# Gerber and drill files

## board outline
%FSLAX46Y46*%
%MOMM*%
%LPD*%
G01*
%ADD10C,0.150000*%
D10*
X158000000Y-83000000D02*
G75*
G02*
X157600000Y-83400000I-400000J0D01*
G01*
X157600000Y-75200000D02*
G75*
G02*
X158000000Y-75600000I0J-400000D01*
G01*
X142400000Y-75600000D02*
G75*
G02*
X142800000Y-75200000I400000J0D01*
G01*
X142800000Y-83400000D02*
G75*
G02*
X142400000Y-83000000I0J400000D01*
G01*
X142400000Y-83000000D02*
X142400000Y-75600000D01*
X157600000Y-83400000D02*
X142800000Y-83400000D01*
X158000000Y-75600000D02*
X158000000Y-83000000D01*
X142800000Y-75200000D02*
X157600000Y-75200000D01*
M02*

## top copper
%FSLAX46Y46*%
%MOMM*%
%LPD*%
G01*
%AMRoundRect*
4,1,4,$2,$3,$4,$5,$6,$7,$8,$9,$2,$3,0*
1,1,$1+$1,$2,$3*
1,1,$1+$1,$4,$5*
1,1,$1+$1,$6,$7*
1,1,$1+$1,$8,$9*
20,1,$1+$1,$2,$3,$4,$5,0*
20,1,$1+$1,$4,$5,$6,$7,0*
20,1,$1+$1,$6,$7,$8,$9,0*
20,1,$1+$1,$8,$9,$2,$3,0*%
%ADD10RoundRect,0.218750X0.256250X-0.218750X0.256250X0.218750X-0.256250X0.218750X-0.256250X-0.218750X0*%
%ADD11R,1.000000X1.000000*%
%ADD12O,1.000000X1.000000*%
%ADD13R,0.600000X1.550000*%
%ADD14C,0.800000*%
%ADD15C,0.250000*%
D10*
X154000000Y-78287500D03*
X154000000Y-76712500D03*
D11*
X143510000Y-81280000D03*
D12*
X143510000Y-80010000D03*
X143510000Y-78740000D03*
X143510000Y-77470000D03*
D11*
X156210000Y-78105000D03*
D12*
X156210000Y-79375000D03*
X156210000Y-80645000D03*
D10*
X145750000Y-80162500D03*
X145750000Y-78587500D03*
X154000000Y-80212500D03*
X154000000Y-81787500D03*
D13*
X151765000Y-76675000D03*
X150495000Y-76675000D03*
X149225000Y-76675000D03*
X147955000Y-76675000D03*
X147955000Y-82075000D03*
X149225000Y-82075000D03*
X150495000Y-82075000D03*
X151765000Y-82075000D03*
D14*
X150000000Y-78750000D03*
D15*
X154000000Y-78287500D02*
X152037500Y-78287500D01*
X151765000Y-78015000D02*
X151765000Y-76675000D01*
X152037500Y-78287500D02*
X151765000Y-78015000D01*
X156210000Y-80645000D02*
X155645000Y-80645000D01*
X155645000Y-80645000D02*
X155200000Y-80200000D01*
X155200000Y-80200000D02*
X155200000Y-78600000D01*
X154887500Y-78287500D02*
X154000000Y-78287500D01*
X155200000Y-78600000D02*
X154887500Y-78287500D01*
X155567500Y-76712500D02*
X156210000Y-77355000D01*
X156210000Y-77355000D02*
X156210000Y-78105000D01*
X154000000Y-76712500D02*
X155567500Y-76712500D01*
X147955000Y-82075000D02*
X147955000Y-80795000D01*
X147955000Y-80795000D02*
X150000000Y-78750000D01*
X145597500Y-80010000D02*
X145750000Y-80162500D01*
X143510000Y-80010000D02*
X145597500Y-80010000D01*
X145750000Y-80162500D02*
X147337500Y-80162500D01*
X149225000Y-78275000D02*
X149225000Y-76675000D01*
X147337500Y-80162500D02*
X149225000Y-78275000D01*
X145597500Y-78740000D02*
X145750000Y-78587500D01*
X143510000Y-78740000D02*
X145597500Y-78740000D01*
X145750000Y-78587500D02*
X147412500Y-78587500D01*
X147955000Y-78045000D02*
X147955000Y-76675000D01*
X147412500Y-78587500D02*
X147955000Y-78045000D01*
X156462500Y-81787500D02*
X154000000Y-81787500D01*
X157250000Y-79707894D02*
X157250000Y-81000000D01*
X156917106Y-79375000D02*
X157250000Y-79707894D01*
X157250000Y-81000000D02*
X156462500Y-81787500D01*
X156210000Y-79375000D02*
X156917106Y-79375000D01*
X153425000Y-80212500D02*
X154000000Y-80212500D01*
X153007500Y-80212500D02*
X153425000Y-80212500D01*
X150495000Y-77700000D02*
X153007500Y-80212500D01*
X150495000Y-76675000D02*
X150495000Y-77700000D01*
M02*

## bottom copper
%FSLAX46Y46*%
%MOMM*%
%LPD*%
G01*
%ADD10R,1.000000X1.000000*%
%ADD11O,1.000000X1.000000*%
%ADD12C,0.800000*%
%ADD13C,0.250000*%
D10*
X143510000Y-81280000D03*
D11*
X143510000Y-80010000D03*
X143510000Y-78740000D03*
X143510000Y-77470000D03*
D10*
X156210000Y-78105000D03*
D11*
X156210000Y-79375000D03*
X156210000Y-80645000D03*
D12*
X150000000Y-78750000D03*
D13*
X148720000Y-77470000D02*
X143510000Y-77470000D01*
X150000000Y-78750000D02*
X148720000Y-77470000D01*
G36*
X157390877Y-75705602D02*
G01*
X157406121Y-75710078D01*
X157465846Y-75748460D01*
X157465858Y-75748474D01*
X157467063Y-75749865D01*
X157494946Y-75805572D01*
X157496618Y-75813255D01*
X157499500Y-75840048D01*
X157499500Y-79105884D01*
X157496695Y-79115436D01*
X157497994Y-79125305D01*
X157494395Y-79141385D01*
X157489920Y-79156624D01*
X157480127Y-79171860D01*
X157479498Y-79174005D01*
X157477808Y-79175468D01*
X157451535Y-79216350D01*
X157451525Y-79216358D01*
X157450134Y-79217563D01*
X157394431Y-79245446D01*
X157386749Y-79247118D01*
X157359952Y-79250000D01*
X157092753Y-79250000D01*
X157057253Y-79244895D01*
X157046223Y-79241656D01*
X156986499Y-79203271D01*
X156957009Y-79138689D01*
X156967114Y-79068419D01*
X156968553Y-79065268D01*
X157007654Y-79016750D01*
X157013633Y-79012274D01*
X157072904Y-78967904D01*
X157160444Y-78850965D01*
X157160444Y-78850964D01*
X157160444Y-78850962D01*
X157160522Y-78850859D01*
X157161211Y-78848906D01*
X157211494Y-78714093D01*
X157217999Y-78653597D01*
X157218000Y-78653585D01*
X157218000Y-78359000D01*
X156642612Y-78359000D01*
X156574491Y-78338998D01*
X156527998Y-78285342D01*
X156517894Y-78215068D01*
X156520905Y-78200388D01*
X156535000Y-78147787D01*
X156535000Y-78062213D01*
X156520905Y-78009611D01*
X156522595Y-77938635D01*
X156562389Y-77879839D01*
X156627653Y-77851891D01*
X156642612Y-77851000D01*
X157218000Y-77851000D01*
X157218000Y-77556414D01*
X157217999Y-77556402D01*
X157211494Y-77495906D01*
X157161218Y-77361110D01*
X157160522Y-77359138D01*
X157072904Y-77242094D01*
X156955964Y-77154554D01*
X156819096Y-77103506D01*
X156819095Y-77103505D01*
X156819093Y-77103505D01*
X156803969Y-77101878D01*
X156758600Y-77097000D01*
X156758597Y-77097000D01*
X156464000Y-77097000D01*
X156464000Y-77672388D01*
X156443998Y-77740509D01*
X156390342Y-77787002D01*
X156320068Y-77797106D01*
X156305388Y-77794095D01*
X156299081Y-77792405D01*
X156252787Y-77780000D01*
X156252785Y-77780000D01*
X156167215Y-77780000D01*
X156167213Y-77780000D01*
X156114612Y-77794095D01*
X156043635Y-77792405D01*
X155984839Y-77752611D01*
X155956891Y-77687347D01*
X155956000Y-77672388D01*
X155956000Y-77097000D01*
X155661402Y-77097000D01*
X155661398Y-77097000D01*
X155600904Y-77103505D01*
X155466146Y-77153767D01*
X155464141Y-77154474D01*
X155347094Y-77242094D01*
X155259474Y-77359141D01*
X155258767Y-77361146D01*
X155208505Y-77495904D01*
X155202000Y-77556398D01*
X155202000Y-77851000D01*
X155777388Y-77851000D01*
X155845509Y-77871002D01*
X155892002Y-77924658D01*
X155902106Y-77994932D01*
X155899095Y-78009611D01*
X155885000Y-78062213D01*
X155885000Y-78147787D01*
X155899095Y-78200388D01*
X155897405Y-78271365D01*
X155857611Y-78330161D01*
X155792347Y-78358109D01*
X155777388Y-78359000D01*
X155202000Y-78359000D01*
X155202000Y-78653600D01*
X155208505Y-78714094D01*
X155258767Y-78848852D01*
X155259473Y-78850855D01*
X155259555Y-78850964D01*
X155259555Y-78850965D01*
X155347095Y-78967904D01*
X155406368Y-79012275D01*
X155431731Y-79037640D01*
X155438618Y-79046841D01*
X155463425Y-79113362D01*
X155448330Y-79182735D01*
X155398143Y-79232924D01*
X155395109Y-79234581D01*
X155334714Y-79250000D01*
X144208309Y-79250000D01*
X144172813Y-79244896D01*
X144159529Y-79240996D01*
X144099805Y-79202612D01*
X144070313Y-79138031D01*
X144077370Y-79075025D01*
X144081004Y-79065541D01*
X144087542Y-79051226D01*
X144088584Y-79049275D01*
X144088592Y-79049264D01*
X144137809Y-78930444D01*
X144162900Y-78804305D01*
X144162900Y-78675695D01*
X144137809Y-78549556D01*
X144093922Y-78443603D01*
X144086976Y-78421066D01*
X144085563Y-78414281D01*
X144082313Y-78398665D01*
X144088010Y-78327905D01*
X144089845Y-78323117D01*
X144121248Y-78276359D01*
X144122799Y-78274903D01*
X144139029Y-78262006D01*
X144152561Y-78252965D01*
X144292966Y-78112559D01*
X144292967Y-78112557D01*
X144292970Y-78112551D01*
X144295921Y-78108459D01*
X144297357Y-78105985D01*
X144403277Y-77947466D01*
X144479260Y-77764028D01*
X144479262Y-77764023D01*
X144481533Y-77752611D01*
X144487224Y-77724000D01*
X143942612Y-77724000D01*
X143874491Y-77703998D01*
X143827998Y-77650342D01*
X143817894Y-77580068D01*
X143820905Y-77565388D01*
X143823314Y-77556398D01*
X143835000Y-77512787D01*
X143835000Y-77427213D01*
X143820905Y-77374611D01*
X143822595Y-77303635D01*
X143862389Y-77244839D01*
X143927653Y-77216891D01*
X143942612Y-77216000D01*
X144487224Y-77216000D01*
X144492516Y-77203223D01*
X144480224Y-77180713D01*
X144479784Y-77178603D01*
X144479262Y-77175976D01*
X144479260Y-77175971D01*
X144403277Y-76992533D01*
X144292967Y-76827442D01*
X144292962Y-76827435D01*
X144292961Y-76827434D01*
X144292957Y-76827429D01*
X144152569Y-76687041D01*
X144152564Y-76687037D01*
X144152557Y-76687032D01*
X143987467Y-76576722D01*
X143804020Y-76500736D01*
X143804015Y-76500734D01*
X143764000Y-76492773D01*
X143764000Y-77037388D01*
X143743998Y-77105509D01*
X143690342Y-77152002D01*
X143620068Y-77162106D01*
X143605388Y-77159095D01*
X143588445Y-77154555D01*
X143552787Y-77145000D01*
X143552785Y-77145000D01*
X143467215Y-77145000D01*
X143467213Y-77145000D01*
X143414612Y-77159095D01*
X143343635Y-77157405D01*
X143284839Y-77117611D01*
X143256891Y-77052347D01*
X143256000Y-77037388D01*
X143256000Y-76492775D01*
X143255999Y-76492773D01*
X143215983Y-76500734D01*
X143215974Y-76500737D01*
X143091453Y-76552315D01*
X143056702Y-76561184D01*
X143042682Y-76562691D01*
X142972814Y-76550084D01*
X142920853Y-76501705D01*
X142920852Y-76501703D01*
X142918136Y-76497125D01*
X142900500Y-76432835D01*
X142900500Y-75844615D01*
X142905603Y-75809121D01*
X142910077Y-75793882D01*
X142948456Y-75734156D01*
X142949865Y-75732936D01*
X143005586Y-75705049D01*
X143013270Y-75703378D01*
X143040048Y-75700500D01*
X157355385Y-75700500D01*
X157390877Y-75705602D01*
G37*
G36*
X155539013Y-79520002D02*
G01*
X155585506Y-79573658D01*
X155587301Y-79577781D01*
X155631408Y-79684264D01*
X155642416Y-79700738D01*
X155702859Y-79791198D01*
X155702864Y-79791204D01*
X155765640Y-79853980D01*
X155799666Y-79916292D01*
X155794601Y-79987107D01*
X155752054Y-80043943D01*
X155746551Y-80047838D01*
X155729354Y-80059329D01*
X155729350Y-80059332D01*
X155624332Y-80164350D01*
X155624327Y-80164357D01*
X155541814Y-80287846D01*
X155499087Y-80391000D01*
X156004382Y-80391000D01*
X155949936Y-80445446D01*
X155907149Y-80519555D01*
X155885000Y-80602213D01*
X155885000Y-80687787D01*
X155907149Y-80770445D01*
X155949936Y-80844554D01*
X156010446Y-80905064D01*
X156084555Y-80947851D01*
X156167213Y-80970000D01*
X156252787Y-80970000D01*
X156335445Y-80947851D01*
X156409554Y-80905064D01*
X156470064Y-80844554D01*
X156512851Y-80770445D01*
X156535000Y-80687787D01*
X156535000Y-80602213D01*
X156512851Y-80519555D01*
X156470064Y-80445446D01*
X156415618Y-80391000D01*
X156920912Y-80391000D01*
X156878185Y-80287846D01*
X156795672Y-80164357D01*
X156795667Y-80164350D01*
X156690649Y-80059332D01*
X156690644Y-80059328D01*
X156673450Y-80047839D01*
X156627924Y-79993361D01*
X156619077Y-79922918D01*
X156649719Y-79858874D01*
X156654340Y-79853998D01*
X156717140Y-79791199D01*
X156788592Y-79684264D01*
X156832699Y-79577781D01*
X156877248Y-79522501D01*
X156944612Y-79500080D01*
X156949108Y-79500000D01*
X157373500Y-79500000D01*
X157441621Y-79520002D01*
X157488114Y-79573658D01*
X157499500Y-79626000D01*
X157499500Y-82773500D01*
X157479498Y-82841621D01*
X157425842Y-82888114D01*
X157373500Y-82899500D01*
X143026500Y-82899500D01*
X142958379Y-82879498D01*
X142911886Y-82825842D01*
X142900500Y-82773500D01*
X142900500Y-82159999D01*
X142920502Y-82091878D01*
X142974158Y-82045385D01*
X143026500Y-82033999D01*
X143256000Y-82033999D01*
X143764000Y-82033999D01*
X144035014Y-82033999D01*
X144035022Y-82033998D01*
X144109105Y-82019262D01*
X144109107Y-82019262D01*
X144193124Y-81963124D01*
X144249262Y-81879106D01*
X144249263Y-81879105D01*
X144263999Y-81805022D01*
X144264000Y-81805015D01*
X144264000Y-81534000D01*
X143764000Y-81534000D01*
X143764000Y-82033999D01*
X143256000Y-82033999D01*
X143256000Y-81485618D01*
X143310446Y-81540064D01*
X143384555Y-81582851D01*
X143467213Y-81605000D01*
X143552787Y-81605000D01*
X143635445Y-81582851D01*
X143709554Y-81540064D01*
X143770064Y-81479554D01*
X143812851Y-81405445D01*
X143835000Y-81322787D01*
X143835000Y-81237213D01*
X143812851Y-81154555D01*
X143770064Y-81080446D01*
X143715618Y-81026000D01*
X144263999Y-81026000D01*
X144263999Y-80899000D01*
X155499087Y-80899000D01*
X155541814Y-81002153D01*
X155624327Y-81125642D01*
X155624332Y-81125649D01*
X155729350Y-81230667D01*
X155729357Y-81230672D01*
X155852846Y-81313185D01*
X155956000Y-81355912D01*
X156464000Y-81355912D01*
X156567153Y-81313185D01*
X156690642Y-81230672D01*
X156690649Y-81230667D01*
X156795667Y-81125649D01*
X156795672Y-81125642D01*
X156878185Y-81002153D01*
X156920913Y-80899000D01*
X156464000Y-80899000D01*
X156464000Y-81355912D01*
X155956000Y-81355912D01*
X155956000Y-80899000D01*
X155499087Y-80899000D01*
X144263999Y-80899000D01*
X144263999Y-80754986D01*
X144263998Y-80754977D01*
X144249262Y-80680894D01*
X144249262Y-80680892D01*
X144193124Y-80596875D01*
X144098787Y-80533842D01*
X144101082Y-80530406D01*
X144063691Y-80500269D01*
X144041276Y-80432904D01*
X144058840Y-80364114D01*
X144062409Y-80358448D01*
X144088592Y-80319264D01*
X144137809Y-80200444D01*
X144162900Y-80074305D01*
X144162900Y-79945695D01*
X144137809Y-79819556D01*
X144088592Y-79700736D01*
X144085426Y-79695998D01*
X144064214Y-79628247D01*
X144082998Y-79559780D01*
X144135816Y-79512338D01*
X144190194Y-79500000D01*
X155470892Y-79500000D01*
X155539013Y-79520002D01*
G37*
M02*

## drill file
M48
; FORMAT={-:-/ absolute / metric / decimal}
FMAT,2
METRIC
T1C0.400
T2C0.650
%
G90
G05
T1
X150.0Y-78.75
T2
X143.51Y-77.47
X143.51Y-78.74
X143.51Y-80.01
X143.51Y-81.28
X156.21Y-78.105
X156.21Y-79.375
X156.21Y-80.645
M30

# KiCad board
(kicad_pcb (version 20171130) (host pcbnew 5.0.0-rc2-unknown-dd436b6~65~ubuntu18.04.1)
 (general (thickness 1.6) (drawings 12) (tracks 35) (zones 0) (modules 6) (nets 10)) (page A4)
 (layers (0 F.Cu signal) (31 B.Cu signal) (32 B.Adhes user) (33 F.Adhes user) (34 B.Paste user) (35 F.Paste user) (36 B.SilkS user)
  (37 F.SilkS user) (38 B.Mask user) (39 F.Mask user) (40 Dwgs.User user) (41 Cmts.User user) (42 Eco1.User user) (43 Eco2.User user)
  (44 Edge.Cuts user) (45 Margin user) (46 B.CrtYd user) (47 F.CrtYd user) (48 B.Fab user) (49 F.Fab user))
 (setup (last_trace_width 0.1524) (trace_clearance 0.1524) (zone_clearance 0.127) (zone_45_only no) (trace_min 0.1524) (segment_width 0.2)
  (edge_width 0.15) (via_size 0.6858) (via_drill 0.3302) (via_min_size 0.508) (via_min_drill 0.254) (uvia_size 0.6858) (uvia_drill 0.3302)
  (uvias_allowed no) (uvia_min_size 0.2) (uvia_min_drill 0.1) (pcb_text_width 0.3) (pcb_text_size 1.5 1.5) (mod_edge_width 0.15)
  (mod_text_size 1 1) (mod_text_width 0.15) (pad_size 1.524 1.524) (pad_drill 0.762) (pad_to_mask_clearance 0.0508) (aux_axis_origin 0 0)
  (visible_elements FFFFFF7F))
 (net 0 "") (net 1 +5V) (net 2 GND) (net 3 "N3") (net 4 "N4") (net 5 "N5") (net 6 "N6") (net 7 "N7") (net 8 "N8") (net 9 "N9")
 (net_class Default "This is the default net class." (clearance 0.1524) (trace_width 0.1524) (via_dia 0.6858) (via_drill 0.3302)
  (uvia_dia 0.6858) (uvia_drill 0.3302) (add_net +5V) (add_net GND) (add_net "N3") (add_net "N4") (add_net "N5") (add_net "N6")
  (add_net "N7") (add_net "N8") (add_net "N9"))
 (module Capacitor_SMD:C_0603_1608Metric (layer F.Cu) (at 154 77.5 90)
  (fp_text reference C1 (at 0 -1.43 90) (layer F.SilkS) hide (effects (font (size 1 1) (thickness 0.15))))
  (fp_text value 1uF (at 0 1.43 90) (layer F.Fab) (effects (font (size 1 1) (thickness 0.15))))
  (pad 1 smd roundrect (at -0.7875 0 90) (size 0.875 0.95) (layers F.Cu F.Paste F.Mask) (roundrect_rratio 0.25) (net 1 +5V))
  (pad 2 smd roundrect (at 0.7875 0 90) (size 0.875 0.95) (layers F.Cu F.Paste F.Mask) (roundrect_rratio 0.25) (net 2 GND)))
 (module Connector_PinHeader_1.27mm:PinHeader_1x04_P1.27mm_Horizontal (layer F.Cu) (at 143.51 81.28 180)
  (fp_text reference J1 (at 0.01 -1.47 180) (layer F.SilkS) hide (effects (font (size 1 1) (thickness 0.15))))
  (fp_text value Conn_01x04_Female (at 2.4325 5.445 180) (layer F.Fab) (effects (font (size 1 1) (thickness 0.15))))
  (pad 1 thru_hole rect (at 0 0 180) (size 1 1) (drill 0.65) (layers *.Cu *.Mask) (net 1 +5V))
  (pad 2 thru_hole oval (at 0 1.27 180) (size 1 1) (drill 0.65) (layers *.Cu *.Mask) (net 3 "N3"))
  (pad 3 thru_hole oval (at 0 2.54 180) (size 1 1) (drill 0.65) (layers *.Cu *.Mask) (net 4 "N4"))
  (pad 4 thru_hole oval (at 0 3.81 180) (size 1 1) (drill 0.65) (layers *.Cu *.Mask) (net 2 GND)))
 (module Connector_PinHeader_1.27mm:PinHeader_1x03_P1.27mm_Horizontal (layer F.Cu) (at 156.21 78.105)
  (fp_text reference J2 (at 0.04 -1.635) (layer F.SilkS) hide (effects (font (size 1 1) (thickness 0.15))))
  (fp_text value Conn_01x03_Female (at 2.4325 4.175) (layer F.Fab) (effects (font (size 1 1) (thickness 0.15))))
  (pad 1 thru_hole rect (at 0 0) (size 1 1) (drill 0.65) (layers *.Cu *.Mask) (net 2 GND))
  (pad 2 thru_hole oval (at 0 1.27) (size 1 1) (drill 0.65) (layers *.Cu *.Mask) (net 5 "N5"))
  (pad 3 thru_hole oval (at 0 2.54) (size 1 1) (drill 0.65) (layers *.Cu *.Mask) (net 1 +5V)))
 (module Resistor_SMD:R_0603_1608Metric (layer F.Cu) (at 145.75 79.375 90)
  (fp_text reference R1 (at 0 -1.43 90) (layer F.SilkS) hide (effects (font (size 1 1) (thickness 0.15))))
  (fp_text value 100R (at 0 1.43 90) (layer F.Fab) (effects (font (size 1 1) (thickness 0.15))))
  (pad 1 smd roundrect (at -0.7875 0 90) (size 0.875 0.95) (layers F.Cu F.Paste F.Mask) (roundrect_rratio 0.25) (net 3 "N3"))
  (pad 2 smd roundrect (at 0.7875 0 90) (size 0.875 0.95) (layers F.Cu F.Paste F.Mask) (roundrect_rratio 0.25) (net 4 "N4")))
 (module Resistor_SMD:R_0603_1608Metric (layer F.Cu) (at 154 81 90)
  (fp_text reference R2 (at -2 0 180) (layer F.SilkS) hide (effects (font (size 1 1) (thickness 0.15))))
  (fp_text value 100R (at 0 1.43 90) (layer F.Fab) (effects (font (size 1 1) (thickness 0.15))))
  (pad 2 smd roundrect (at 0.7875 0 90) (size 0.875 0.95) (layers F.Cu F.Paste F.Mask) (roundrect_rratio 0.25) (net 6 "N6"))
  (pad 1 smd roundrect (at -0.7875 0 90) (size 0.875 0.95) (layers F.Cu F.Paste F.Mask) (roundrect_rratio 0.25) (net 5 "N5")))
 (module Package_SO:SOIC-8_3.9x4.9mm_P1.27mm (layer F.Cu) (at 149.86 79.375 270)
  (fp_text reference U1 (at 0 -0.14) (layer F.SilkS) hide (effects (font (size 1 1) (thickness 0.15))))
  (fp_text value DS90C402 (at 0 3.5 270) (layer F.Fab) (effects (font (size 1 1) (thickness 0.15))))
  (pad 1 smd rect (at -2.7 -1.905 270) (size 1.55 0.6) (layers F.Cu F.Paste F.Mask) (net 1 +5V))
  (pad 2 smd rect (at -2.7 -0.635 270) (size 1.55 0.6) (layers F.Cu F.Paste F.Mask) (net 6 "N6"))
  (pad 3 smd rect (at -2.7 0.635 270) (size 1.55 0.6) (layers F.Cu F.Paste F.Mask) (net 3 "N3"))
  (pad 4 smd rect (at -2.7 1.905 270) (size 1.55 0.6) (layers F.Cu F.Paste F.Mask) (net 4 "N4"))
  (pad 5 smd rect (at 2.7 1.905 270) (size 1.55 0.6) (layers F.Cu F.Paste F.Mask) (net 2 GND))
  (pad 6 smd rect (at 2.7 0.635 270) (size 1.55 0.6) (layers F.Cu F.Paste F.Mask) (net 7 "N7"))
  (pad 7 smd rect (at 2.7 -0.635 270) (size 1.55 0.6) (layers F.Cu F.Paste F.Mask) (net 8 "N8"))
  (pad 8 smd rect (at 2.7 -1.905 270) (size 1.55 0.6) (layers F.Cu F.Paste F.Mask) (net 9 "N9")))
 (gr_arc (start 157.6 83) (end 157.6 83.4) (angle -90) (layer Edge.Cuts) (width 0.15))
 (gr_arc (start 157.6 75.6) (end 158 75.6) (angle -90) (layer Edge.Cuts) (width 0.15))
 (gr_arc (start 142.8 75.6) (end 142.8 75.2) (angle -90) (layer Edge.Cuts) (width 0.15))
 (gr_arc (start 142.8 83) (end 142.4 83) (angle -90) (layer Edge.Cuts) (width 0.15))
 (gr_line (start 142.4 83) (end 142.4 75.6) (layer Edge.Cuts) (width 0.15))
 (gr_line (start 157.6 83.4) (end 142.8 83.4) (layer Edge.Cuts) (width 0.15))
 (gr_line (start 158 75.6) (end 158 83) (layer Edge.Cuts) (width 0.15))
 (gr_line (start 142.8 75.2) (end 157.6 75.2) (layer Edge.Cuts) (width 0.15))
 (segment (start 154 78.2875) (end 152.0375 78.2875) (width 0.25) (layer F.Cu) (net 1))
 (segment (start 151.765 78.015) (end 151.765 76.675) (width 0.25) (layer F.Cu) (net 1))
 (segment (start 152.0375 78.2875) (end 151.765 78.015) (width 0.25) (layer F.Cu) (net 1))
 (segment (start 156.21 80.645) (end 155.645 80.645) (width 0.25) (layer F.Cu) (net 1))
 (segment (start 155.645 80.645) (end 155.2 80.2) (width 0.25) (layer F.Cu) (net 1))
 (segment (start 155.2 80.2) (end 155.2 78.6) (width 0.25) (layer F.Cu) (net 1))
 (segment (start 154.8875 78.2875) (end 154 78.2875) (width 0.25) (layer F.Cu) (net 1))
 (segment (start 155.2 78.6) (end 154.8875 78.2875) (width 0.25) (layer F.Cu) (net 1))
 (segment (start 155.5675 76.7125) (end 156.21 77.355) (width 0.25) (layer F.Cu) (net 2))
 (segment (start 156.21 77.355) (end 156.21 78.105) (width 0.25) (layer F.Cu) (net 2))
 (segment (start 154 76.7125) (end 155.5675 76.7125) (width 0.25) (layer F.Cu) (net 2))
 (via (at 150 78.75) (size 0.8) (drill 0.4) (layers F.Cu B.Cu) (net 2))
 (segment (start 147.955 82.075) (end 147.955 80.795) (width 0.25) (layer F.Cu) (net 2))
 (segment (start 147.955 80.795) (end 150 78.75) (width 0.25) (layer F.Cu) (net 2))
 (segment (start 148.72 77.47) (end 143.51 77.47) (width 0.25) (layer B.Cu) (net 2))
 (segment (start 150 78.75) (end 148.72 77.47) (width 0.25) (layer B.Cu) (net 2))
 (segment (start 145.5975 80.01) (end 145.75 80.1625) (width 0.25) (layer F.Cu) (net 3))
 (segment (start 143.51 80.01) (end 145.5975 80.01) (width 0.25) (layer F.Cu) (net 3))
 (segment (start 145.75 80.1625) (end 147.3375 80.1625) (width 0.25) (layer F.Cu) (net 3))
 (segment (start 149.225 78.275) (end 149.225 76.675) (width 0.25) (layer F.Cu) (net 3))
 (segment (start 147.3375 80.1625) (end 149.225 78.275) (width 0.25) (layer F.Cu) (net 3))
 (segment (start 145.5975 78.74) (end 145.75 78.5875) (width 0.25) (layer F.Cu) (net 4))
 (segment (start 143.51 78.74) (end 145.5975 78.74) (width 0.25) (layer F.Cu) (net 4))
 (segment (start 145.75 78.5875) (end 147.4125 78.5875) (width 0.25) (layer F.Cu) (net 4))
 (segment (start 147.955 78.045) (end 147.955 76.675) (width 0.25) (layer F.Cu) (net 4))
 (segment (start 147.4125 78.5875) (end 147.955 78.045) (width 0.25) (layer F.Cu) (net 4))
 (segment (start 156.4625 81.7875) (end 154 81.7875) (width 0.25) (layer F.Cu) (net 5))
 (segment (start 157.25 79.707894) (end 157.25 81) (width 0.25) (layer F.Cu) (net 5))
 (segment (start 156.917106 79.375) (end 157.25 79.707894) (width 0.25) (layer F.Cu) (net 5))
 (segment (start 157.25 81) (end 156.4625 81.7875) (width 0.25) (layer F.Cu) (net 5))
 (segment (start 156.21 79.375) (end 156.917106 79.375) (width 0.25) (layer F.Cu) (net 5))
 (segment (start 153.425 80.2125) (end 154 80.2125) (width 0.25) (layer F.Cu) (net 6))
 (segment (start 153.0075 80.2125) (end 153.425 80.2125) (width 0.25) (layer F.Cu) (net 6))
 (segment (start 150.495 77.7) (end 153.0075 80.2125) (width 0.25) (layer F.Cu) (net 6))
 (segment (start 150.495 76.675) (end 150.495 77.7) (width 0.25) (layer F.Cu) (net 6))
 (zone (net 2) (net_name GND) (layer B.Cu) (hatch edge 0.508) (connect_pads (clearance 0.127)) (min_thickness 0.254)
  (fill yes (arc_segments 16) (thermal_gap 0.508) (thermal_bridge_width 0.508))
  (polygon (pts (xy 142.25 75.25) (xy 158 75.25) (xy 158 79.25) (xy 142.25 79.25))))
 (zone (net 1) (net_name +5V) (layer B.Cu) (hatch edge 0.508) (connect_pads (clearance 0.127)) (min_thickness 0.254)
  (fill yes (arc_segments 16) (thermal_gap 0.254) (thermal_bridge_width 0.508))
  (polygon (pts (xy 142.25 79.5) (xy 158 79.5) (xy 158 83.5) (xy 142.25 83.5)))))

